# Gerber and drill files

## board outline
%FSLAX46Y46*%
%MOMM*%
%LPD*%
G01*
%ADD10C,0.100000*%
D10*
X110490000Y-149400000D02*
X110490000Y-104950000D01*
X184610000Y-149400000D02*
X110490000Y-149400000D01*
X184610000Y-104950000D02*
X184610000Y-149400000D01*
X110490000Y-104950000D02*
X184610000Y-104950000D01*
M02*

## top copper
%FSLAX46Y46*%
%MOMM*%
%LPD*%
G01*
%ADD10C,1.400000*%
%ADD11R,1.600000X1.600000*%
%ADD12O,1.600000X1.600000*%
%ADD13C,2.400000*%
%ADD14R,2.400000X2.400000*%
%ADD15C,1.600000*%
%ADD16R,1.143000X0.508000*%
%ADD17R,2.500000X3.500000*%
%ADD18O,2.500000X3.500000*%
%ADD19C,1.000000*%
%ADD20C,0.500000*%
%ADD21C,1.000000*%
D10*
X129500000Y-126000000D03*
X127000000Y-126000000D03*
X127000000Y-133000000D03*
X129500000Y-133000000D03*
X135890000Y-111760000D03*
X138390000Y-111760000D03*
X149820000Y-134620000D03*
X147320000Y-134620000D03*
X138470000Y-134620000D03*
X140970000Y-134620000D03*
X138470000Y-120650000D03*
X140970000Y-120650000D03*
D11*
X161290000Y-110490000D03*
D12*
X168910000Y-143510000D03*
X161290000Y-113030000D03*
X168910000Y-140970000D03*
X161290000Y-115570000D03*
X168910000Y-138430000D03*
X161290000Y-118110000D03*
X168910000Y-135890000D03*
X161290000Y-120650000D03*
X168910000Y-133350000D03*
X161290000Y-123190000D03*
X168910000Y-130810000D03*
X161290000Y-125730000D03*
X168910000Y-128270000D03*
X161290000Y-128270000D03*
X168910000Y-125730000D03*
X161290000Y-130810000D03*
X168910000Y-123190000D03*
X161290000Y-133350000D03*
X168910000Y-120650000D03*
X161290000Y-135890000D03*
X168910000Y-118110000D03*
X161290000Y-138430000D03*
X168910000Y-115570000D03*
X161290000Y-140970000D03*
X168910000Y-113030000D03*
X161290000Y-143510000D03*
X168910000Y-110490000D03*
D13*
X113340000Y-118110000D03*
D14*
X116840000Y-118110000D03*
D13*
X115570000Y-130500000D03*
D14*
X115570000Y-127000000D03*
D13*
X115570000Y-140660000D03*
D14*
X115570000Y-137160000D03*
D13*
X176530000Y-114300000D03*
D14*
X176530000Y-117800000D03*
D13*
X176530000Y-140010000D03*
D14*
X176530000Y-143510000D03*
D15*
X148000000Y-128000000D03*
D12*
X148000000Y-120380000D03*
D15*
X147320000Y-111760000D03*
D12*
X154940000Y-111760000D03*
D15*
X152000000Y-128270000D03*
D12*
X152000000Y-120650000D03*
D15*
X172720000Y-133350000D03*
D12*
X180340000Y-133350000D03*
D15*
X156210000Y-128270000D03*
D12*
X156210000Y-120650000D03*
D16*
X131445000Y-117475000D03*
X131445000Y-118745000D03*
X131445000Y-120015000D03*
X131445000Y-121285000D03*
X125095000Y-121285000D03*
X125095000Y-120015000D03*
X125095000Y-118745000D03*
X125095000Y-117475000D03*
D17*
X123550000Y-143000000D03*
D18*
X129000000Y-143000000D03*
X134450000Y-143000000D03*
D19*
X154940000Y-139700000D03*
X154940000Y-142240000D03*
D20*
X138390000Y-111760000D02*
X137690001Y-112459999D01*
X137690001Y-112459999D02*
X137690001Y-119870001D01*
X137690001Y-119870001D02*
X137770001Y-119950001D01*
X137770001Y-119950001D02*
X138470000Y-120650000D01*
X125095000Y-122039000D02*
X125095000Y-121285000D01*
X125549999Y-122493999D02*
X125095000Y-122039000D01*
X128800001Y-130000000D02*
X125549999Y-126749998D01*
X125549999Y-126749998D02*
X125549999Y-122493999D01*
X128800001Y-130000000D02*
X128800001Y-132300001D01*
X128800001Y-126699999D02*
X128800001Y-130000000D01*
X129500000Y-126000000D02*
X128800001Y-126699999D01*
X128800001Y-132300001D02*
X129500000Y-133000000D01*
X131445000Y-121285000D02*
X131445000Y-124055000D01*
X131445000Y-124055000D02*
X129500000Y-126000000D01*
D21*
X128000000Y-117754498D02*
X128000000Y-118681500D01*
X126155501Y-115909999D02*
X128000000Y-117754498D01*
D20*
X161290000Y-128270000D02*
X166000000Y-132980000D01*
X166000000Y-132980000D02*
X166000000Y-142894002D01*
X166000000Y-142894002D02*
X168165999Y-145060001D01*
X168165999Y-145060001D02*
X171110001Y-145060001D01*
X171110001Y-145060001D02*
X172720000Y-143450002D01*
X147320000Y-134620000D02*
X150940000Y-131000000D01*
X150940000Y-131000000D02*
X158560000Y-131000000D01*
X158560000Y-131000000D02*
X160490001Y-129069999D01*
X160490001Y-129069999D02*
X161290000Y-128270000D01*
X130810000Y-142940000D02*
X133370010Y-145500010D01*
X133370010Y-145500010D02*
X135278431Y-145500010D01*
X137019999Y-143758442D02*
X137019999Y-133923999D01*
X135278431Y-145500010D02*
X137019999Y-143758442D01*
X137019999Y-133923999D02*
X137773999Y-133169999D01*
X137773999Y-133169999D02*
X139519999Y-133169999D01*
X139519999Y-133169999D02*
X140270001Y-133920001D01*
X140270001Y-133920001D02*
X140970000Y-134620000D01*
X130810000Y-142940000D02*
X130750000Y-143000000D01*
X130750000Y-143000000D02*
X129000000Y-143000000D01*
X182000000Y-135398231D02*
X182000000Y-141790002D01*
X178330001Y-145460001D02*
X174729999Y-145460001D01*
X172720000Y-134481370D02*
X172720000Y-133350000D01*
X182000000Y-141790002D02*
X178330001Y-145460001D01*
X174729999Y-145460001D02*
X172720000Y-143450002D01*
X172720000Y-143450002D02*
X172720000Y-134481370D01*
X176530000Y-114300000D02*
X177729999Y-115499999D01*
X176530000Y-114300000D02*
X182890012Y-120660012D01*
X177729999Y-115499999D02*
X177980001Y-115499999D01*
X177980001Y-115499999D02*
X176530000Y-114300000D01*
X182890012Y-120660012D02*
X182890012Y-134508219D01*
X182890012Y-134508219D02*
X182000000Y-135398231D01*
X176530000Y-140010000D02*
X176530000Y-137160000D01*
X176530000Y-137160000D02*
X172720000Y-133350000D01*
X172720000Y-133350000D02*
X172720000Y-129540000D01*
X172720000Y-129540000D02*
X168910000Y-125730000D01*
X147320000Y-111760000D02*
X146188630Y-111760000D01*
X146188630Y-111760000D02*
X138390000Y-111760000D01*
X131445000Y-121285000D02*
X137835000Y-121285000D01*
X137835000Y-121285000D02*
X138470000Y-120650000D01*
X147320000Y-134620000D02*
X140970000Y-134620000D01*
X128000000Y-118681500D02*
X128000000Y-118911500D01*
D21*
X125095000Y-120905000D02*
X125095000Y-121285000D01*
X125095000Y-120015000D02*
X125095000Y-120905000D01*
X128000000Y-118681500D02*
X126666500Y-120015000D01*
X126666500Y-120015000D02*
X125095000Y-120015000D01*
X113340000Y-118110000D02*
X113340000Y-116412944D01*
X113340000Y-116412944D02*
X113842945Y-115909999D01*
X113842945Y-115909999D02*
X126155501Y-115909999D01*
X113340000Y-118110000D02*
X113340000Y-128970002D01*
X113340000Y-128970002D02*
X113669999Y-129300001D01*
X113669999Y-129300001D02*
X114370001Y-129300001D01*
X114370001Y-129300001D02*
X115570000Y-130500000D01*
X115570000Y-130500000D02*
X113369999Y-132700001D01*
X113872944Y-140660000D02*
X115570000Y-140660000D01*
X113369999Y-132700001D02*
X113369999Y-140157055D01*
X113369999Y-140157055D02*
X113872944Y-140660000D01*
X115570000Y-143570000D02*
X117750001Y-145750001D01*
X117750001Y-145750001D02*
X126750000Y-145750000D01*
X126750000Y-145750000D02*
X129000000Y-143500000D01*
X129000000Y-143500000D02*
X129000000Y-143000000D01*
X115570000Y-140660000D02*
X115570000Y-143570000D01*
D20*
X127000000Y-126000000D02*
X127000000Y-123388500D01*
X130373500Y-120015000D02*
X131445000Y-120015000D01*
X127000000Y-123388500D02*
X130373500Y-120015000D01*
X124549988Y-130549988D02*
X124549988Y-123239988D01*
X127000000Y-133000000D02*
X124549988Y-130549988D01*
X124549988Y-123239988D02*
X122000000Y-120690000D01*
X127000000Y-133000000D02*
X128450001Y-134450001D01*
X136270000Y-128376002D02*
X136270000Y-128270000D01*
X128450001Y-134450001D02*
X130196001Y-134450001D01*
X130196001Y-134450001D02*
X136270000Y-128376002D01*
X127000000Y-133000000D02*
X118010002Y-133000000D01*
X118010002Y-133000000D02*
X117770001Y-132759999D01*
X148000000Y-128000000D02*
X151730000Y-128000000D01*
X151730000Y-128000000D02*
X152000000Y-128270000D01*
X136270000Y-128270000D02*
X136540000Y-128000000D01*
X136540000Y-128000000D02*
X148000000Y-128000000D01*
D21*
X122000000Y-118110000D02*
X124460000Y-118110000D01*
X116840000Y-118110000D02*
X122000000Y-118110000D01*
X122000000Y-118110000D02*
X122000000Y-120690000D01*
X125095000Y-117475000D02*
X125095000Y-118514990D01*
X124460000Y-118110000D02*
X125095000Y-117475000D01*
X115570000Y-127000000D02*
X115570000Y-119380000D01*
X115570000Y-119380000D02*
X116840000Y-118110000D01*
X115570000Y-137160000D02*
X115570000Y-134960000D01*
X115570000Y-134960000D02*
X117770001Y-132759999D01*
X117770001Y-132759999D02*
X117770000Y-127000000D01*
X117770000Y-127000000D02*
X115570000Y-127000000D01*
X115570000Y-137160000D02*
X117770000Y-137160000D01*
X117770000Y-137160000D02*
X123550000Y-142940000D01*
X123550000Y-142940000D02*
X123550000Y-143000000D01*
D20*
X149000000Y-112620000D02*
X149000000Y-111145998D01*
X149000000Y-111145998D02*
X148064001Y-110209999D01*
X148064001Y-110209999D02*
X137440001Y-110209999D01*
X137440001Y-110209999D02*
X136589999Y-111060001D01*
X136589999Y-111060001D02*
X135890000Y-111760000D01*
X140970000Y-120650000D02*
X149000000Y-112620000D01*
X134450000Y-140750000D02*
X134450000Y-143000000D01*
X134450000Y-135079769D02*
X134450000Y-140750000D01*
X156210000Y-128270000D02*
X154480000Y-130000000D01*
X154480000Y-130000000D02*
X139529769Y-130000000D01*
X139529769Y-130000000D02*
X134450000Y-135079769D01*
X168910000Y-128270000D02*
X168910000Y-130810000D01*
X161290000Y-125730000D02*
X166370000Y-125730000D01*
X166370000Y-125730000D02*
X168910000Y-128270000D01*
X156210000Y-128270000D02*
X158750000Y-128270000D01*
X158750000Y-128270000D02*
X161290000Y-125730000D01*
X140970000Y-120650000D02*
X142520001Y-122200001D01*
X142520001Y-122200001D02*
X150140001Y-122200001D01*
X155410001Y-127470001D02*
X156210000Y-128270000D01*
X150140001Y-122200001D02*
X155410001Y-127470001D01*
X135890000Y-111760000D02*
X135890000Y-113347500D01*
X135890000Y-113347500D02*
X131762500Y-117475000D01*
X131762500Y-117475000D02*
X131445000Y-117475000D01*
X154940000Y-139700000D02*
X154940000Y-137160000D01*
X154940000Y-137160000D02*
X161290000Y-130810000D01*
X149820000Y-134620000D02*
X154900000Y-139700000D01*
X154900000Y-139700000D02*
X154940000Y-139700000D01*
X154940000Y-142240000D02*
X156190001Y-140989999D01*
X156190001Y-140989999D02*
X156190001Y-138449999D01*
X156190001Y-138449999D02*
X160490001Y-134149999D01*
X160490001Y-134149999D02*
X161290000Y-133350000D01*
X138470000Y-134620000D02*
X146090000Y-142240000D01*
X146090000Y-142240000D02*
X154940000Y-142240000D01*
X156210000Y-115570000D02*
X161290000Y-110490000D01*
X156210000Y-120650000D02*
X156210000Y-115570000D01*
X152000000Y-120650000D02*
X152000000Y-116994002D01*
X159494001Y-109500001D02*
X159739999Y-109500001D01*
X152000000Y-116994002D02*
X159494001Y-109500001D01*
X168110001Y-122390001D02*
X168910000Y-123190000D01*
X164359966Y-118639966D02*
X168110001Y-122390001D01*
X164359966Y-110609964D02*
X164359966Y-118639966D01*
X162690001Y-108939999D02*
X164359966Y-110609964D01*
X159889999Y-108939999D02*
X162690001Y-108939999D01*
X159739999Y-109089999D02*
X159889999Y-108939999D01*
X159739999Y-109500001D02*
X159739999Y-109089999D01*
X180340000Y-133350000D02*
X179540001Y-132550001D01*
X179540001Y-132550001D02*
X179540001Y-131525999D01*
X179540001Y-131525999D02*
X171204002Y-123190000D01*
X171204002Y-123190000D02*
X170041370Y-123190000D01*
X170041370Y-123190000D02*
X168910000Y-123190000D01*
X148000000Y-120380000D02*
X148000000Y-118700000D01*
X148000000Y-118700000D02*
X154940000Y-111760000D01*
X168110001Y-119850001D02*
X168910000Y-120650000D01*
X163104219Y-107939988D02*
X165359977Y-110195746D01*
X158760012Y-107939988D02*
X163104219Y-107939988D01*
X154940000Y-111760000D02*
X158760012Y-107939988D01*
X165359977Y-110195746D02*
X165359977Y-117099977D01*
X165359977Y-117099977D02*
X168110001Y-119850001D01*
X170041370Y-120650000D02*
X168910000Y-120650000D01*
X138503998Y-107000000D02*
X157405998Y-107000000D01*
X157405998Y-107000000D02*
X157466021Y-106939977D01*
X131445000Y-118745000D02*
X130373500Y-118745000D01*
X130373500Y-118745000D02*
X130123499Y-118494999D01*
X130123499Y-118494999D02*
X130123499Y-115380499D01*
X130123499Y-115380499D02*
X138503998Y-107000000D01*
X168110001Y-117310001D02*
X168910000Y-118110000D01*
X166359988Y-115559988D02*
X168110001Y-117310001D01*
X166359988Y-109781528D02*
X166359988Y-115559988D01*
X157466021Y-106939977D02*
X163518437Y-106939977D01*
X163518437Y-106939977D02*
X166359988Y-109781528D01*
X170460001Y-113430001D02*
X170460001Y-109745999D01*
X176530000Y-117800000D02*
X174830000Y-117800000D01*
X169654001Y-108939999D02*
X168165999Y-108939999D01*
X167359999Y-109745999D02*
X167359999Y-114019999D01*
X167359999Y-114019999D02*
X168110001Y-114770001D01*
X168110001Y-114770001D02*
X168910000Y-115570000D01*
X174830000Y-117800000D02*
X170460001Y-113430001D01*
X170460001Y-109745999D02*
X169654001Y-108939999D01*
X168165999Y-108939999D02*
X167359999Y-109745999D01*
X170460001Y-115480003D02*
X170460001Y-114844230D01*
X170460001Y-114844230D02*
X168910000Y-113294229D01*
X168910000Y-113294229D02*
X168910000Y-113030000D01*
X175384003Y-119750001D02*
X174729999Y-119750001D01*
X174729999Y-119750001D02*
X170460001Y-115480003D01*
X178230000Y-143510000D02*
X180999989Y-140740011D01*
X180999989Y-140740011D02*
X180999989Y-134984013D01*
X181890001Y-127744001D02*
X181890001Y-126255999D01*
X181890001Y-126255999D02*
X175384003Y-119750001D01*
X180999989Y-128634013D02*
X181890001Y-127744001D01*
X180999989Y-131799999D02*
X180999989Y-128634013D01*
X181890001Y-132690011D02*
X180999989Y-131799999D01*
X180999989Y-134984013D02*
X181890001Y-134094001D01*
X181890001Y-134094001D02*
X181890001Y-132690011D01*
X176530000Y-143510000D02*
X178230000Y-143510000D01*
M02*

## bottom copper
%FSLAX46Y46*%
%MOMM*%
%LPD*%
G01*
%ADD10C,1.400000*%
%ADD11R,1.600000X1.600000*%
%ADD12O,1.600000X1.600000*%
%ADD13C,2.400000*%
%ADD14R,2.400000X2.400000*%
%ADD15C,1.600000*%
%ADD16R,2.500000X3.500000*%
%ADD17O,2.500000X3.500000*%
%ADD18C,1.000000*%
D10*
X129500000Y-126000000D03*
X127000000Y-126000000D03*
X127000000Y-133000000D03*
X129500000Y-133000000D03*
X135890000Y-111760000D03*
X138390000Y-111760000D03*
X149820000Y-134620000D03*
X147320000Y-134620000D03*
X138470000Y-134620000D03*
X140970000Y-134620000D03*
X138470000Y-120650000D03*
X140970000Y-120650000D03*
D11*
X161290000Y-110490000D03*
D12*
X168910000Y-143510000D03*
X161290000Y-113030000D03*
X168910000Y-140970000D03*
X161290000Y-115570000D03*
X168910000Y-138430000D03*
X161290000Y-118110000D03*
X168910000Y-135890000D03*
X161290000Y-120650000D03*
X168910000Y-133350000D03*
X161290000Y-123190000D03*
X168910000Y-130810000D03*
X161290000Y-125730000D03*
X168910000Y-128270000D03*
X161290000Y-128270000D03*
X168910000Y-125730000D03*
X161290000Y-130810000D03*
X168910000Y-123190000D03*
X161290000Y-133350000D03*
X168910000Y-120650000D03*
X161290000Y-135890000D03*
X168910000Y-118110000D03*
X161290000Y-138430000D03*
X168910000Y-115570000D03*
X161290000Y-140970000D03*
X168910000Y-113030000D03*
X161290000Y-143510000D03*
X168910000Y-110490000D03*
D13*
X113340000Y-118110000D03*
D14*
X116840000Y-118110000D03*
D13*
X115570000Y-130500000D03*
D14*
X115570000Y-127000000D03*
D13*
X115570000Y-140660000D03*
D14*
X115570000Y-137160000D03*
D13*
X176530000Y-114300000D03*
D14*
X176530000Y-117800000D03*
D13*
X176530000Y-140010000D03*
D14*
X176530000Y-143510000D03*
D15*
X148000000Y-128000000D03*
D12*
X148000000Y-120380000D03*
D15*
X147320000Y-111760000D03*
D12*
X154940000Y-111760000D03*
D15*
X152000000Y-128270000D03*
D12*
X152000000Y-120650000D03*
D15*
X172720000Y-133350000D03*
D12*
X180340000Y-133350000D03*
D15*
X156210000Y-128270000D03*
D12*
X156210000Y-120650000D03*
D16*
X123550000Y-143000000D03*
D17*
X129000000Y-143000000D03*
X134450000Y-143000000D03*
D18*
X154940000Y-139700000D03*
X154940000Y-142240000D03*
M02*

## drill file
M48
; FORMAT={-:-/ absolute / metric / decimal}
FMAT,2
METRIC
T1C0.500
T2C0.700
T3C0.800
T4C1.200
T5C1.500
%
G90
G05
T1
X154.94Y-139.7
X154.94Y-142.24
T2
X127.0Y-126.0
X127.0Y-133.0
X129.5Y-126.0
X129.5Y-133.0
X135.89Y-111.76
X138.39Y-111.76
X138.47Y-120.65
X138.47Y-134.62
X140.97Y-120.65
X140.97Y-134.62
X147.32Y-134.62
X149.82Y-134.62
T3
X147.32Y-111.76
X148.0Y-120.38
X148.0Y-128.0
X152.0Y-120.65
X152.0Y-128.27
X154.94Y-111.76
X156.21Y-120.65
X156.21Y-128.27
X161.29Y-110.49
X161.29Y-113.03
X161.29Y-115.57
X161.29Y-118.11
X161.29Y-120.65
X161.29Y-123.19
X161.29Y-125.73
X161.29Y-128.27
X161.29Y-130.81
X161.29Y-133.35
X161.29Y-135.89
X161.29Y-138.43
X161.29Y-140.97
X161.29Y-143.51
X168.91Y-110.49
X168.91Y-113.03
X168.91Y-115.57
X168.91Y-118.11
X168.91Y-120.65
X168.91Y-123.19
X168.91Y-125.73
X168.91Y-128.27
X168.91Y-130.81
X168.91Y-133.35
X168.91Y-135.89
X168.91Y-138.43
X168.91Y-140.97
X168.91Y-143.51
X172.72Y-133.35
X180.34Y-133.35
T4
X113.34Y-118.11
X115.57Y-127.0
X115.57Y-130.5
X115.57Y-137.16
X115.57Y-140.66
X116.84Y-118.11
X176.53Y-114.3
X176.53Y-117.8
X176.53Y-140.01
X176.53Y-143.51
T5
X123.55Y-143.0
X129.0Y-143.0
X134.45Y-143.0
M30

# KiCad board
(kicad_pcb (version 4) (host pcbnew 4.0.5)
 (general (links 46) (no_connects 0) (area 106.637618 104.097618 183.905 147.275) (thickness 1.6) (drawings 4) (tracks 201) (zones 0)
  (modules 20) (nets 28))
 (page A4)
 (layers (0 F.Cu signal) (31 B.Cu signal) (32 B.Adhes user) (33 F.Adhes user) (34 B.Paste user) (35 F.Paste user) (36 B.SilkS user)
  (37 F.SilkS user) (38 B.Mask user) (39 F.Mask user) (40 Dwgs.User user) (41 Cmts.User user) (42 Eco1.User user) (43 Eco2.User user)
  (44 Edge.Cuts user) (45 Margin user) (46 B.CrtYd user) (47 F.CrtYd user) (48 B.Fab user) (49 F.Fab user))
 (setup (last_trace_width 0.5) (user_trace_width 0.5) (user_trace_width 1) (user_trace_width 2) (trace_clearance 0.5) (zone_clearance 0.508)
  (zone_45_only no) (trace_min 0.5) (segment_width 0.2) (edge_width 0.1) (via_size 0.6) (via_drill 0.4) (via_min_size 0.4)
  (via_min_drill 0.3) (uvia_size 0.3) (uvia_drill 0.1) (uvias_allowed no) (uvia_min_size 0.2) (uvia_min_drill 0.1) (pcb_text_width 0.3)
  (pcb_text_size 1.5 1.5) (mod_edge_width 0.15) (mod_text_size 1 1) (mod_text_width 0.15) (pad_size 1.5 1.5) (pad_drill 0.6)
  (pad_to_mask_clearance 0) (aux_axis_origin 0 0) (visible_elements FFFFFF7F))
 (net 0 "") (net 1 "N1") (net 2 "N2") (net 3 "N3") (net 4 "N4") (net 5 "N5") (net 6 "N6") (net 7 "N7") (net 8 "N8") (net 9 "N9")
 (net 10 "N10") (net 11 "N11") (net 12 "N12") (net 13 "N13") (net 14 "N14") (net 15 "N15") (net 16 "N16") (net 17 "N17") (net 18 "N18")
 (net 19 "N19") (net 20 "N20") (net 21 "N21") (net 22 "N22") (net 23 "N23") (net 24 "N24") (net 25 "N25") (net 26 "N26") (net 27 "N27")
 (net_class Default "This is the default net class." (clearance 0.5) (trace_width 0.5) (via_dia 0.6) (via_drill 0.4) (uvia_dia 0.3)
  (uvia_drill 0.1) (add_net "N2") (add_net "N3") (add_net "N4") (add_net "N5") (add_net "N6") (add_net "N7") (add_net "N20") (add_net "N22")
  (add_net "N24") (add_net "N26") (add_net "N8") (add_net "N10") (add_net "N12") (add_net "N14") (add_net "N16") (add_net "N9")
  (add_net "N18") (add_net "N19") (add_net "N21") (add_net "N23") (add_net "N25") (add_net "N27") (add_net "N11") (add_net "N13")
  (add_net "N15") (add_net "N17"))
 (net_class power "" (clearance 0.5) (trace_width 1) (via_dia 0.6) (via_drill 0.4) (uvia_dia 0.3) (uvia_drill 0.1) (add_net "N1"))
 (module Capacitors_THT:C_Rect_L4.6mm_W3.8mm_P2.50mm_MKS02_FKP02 (layer F.Cu) (at 129.5 126 180)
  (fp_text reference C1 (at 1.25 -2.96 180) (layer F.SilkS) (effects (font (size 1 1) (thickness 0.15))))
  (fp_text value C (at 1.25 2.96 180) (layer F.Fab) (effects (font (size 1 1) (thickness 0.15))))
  (pad 1 thru_hole circle (at 0 0 180) (size 1.4 1.4) (drill 0.7) (layers *.Cu *.Mask) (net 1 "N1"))
  (pad 2 thru_hole circle (at 2.5 0 180) (size 1.4 1.4) (drill 0.7) (layers *.Cu *.Mask) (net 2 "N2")))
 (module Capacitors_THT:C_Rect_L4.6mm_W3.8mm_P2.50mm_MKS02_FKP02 (layer F.Cu) (at 127 133)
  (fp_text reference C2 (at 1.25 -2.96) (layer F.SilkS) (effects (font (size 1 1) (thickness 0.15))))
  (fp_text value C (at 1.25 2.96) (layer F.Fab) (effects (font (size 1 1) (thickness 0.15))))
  (pad 1 thru_hole circle (at 0 0) (size 1.4 1.4) (drill 0.7) (layers *.Cu *.Mask) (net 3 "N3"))
  (pad 2 thru_hole circle (at 2.5 0) (size 1.4 1.4) (drill 0.7) (layers *.Cu *.Mask) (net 1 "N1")))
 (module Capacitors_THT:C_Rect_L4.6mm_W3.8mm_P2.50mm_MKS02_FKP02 (layer F.Cu) (at 135.89 111.76)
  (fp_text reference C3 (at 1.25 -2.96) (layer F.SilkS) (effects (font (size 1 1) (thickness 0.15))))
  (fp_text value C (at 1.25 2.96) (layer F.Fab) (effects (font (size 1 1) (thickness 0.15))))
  (pad 1 thru_hole circle (at 0 0) (size 1.4 1.4) (drill 0.7) (layers *.Cu *.Mask) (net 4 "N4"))
  (pad 2 thru_hole circle (at 2.5 0) (size 1.4 1.4) (drill 0.7) (layers *.Cu *.Mask) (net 1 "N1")))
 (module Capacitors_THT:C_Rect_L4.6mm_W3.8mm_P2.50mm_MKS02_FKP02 (layer F.Cu) (at 149.82 134.62 180)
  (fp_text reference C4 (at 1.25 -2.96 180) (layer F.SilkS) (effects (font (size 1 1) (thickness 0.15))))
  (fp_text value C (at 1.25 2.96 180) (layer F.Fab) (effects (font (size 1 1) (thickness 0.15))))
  (pad 1 thru_hole circle (at 0 0 180) (size 1.4 1.4) (drill 0.7) (layers *.Cu *.Mask) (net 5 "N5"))
  (pad 2 thru_hole circle (at 2.5 0 180) (size 1.4 1.4) (drill 0.7) (layers *.Cu *.Mask) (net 1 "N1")))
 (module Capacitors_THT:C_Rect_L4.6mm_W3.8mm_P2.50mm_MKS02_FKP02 (layer F.Cu) (at 138.47 134.62)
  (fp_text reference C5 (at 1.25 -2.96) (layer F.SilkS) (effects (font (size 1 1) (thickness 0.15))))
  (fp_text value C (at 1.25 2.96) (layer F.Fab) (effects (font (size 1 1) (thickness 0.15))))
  (pad 1 thru_hole circle (at 0 0) (size 1.4 1.4) (drill 0.7) (layers *.Cu *.Mask) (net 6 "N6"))
  (pad 2 thru_hole circle (at 2.5 0) (size 1.4 1.4) (drill 0.7) (layers *.Cu *.Mask) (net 1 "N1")))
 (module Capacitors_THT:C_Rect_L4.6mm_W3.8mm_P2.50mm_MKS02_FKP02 (layer F.Cu) (at 138.47 120.65)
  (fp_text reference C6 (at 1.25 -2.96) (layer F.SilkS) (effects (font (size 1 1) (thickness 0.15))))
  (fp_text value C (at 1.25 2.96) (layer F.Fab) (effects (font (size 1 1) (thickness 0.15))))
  (pad 1 thru_hole circle (at 0 0) (size 1.4 1.4) (drill 0.7) (layers *.Cu *.Mask) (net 1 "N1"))
  (pad 2 thru_hole circle (at 2.5 0) (size 1.4 1.4) (drill 0.7) (layers *.Cu *.Mask) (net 4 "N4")))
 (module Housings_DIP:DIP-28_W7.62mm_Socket (layer F.Cu) (at 161.29 110.49)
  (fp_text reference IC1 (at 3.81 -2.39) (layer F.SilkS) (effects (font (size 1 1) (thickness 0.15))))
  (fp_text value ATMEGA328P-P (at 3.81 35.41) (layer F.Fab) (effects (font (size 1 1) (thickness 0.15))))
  (pad 1 thru_hole rect (at 0 0) (size 1.6 1.6) (drill 0.8) (layers *.Cu *.Mask) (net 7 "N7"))
  (pad 15 thru_hole oval (at 7.62 33.02) (size 1.6 1.6) (drill 0.8) (layers *.Cu *.Mask) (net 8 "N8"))
  (pad 2 thru_hole oval (at 0 2.54) (size 1.6 1.6) (drill 0.8) (layers *.Cu *.Mask) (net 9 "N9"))
  (pad 16 thru_hole oval (at 7.62 30.48) (size 1.6 1.6) (drill 0.8) (layers *.Cu *.Mask) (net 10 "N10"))
  (pad 3 thru_hole oval (at 0 5.08) (size 1.6 1.6) (drill 0.8) (layers *.Cu *.Mask) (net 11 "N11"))
  (pad 17 thru_hole oval (at 7.62 27.94) (size 1.6 1.6) (drill 0.8) (layers *.Cu *.Mask) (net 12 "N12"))
  (pad 4 thru_hole oval (at 0 7.62) (size 1.6 1.6) (drill 0.8) (layers *.Cu *.Mask) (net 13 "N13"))
  (pad 18 thru_hole oval (at 7.62 25.4) (size 1.6 1.6) (drill 0.8) (layers *.Cu *.Mask) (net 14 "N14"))
  (pad 5 thru_hole oval (at 0 10.16) (size 1.6 1.6) (drill 0.8) (layers *.Cu *.Mask) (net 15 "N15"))
  (pad 19 thru_hole oval (at 7.62 22.86) (size 1.6 1.6) (drill 0.8) (layers *.Cu *.Mask) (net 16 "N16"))
  (pad 6 thru_hole oval (at 0 12.7) (size 1.6 1.6) (drill 0.8) (layers *.Cu *.Mask) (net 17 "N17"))
  (pad 20 thru_hole oval (at 7.62 20.32) (size 1.6 1.6) (drill 0.8) (layers *.Cu *.Mask) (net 4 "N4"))
  (pad 7 thru_hole oval (at 0 15.24) (size 1.6 1.6) (drill 0.8) (layers *.Cu *.Mask) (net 4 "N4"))
  (pad 21 thru_hole oval (at 7.62 17.78) (size 1.6 1.6) (drill 0.8) (layers *.Cu *.Mask) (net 4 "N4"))
  (pad 8 thru_hole oval (at 0 17.78) (size 1.6 1.6) (drill 0.8) (layers *.Cu *.Mask) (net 1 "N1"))
  (pad 22 thru_hole oval (at 7.62 15.24) (size 1.6 1.6) (drill 0.8) (layers *.Cu *.Mask) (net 1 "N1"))
  (pad 9 thru_hole oval (at 0 20.32) (size 1.6 1.6) (drill 0.8) (layers *.Cu *.Mask) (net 5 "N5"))
  (pad 23 thru_hole oval (at 7.62 12.7) (size 1.6 1.6) (drill 0.8) (layers *.Cu *.Mask) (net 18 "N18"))
  (pad 10 thru_hole oval (at 0 22.86) (size 1.6 1.6) (drill 0.8) (layers *.Cu *.Mask) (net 6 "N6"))
  (pad 24 thru_hole oval (at 7.62 10.16) (size 1.6 1.6) (drill 0.8) (layers *.Cu *.Mask) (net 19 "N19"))
  (pad 11 thru_hole oval (at 0 25.4) (size 1.6 1.6) (drill 0.8) (layers *.Cu *.Mask) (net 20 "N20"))
  (pad 25 thru_hole oval (at 7.62 7.62) (size 1.6 1.6) (drill 0.8) (layers *.Cu *.Mask) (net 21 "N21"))
  (pad 12 thru_hole oval (at 0 27.94) (size 1.6 1.6) (drill 0.8) (layers *.Cu *.Mask) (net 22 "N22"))
  (pad 26 thru_hole oval (at 7.62 5.08) (size 1.6 1.6) (drill 0.8) (layers *.Cu *.Mask) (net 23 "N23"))
  (pad 13 thru_hole oval (at 0 30.48) (size 1.6 1.6) (drill 0.8) (layers *.Cu *.Mask) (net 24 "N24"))
  (pad 27 thru_hole oval (at 7.62 2.54) (size 1.6 1.6) (drill 0.8) (layers *.Cu *.Mask) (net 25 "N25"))
  (pad 14 thru_hole oval (at 0 33.02) (size 1.6 1.6) (drill 0.8) (layers *.Cu *.Mask) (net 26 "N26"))
  (pad 28 thru_hole oval (at 7.62 0) (size 1.6 1.6) (drill 0.8) (layers *.Cu *.Mask) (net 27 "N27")))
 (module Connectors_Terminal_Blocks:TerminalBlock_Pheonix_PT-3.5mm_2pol (layer F.Cu) (at 116.84 118.11 180)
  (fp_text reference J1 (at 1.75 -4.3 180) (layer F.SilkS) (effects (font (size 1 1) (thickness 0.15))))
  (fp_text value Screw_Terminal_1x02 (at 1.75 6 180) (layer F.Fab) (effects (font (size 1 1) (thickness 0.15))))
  (pad 2 thru_hole circle (at 3.5 0 180) (size 2.4 2.4) (drill 1.2) (layers *.Cu *.Mask) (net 1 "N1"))
  (pad 1 thru_hole rect (at 0 0 180) (size 2.4 2.4) (drill 1.2) (layers *.Cu *.Mask) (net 3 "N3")))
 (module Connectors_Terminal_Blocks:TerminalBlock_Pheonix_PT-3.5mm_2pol (layer F.Cu) (at 115.57 127 270)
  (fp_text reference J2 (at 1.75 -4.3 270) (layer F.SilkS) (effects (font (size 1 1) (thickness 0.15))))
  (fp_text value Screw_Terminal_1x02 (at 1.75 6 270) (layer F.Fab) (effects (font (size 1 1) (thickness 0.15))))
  (pad 2 thru_hole circle (at 3.5 0 270) (size 2.4 2.4) (drill 1.2) (layers *.Cu *.Mask) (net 1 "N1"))
  (pad 1 thru_hole rect (at 0 0 270) (size 2.4 2.4) (drill 1.2) (layers *.Cu *.Mask) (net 3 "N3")))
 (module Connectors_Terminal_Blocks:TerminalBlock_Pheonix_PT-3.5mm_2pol (layer F.Cu) (at 115.57 137.16 270)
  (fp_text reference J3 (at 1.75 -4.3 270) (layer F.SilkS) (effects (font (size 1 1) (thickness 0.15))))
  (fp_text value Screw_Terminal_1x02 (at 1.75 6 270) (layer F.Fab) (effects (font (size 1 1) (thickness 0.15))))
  (pad 2 thru_hole circle (at 3.5 0 270) (size 2.4 2.4) (drill 1.2) (layers *.Cu *.Mask) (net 1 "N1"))
  (pad 1 thru_hole rect (at 0 0 270) (size 2.4 2.4) (drill 1.2) (layers *.Cu *.Mask) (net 3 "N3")))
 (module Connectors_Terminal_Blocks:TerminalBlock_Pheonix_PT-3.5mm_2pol (layer F.Cu) (at 176.53 117.8 90)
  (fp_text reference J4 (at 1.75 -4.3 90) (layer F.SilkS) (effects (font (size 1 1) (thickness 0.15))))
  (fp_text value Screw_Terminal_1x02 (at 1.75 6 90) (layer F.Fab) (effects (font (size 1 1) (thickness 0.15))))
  (pad 2 thru_hole circle (at 3.5 0 90) (size 2.4 2.4) (drill 1.2) (layers *.Cu *.Mask) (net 1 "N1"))
  (pad 1 thru_hole rect (at 0 0 90) (size 2.4 2.4) (drill 1.2) (layers *.Cu *.Mask) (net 23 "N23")))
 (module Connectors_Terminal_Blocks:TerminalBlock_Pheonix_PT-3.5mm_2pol (layer F.Cu) (at 176.53 143.51 90)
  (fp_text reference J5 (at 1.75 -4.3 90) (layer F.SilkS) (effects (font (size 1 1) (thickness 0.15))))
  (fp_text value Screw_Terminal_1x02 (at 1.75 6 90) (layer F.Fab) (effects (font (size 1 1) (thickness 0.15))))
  (pad 2 thru_hole circle (at 3.5 0 90) (size 2.4 2.4) (drill 1.2) (layers *.Cu *.Mask) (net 1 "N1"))
  (pad 1 thru_hole rect (at 0 0 90) (size 2.4 2.4) (drill 1.2) (layers *.Cu *.Mask) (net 25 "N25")))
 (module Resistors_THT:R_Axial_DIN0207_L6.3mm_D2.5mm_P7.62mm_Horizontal (layer F.Cu) (at 148 128 90)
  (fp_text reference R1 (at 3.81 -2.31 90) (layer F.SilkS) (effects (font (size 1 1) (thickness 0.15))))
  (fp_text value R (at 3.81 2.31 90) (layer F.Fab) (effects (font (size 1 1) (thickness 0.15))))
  (pad 1 thru_hole circle (at 0 0 90) (size 1.6 1.6) (drill 0.8) (layers *.Cu *.Mask) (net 3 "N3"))
  (pad 2 thru_hole oval (at 7.62 0 90) (size 1.6 1.6) (drill 0.8) (layers *.Cu *.Mask) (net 19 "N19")))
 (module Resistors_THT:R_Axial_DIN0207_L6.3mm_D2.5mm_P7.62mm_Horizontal (layer F.Cu) (at 147.32 111.76)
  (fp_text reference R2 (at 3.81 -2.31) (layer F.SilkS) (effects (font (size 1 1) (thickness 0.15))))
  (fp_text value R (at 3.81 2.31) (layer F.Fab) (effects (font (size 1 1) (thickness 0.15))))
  (pad 1 thru_hole circle (at 0 0) (size 1.6 1.6) (drill 0.8) (layers *.Cu *.Mask) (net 1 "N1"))
  (pad 2 thru_hole oval (at 7.62 0) (size 1.6 1.6) (drill 0.8) (layers *.Cu *.Mask) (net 19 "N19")))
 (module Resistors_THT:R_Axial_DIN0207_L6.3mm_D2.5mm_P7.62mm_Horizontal (layer F.Cu) (at 152 128.27 90)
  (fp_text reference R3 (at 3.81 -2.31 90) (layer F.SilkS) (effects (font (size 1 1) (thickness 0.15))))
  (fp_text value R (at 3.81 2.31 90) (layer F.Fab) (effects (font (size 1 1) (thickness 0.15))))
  (pad 1 thru_hole circle (at 0 0 90) (size 1.6 1.6) (drill 0.8) (layers *.Cu *.Mask) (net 3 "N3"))
  (pad 2 thru_hole oval (at 7.62 0 90) (size 1.6 1.6) (drill 0.8) (layers *.Cu *.Mask) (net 18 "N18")))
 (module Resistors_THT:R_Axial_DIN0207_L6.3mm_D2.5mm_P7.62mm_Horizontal (layer F.Cu) (at 172.72 133.35)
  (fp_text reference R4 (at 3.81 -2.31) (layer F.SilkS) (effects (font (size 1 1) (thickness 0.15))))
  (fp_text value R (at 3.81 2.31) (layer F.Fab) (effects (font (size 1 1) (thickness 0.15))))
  (pad 1 thru_hole circle (at 0 0) (size 1.6 1.6) (drill 0.8) (layers *.Cu *.Mask) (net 1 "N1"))
  (pad 2 thru_hole oval (at 7.62 0) (size 1.6 1.6) (drill 0.8) (layers *.Cu *.Mask) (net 18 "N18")))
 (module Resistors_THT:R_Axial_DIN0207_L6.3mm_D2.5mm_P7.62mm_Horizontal (layer F.Cu) (at 156.21 128.27 90)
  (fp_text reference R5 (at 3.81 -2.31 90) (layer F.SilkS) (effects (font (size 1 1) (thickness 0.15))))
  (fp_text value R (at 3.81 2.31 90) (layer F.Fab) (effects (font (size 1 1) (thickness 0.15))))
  (pad 1 thru_hole circle (at 0 0 90) (size 1.6 1.6) (drill 0.8) (layers *.Cu *.Mask) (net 4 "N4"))
  (pad 2 thru_hole oval (at 7.62 0 90) (size 1.6 1.6) (drill 0.8) (layers *.Cu *.Mask) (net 7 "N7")))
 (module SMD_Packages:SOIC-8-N (layer F.Cu) (at 128.27 119.38 270)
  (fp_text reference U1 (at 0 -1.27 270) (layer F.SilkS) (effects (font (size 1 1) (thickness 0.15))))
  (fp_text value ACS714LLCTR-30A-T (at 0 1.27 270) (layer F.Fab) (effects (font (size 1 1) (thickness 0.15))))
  (pad 8 smd rect (at -1.905 -3.175 270) (size 0.508 1.143) (layers F.Cu F.Paste F.Mask) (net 4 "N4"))
  (pad 7 smd rect (at -0.635 -3.175 270) (size 0.508 1.143) (layers F.Cu F.Paste F.Mask) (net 21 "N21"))
  (pad 6 smd rect (at 0.635 -3.175 270) (size 0.508 1.143) (layers F.Cu F.Paste F.Mask) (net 2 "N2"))
  (pad 5 smd rect (at 1.905 -3.175 270) (size 0.508 1.143) (layers F.Cu F.Paste F.Mask) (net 1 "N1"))
  (pad 4 smd rect (at 1.905 3.175 270) (size 0.508 1.143) (layers F.Cu F.Paste F.Mask) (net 1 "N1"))
  (pad 3 smd rect (at 0.635 3.175 270) (size 0.508 1.143) (layers F.Cu F.Paste F.Mask) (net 1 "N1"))
  (pad 2 smd rect (at -0.635 3.175 270) (size 0.508 1.143) (layers F.Cu F.Paste F.Mask) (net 3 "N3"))
  (pad 1 smd rect (at -1.905 3.175 270) (size 0.508 1.143) (layers F.Cu F.Paste F.Mask) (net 3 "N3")))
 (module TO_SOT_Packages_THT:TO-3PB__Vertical (layer F.Cu) (at 123.55 143)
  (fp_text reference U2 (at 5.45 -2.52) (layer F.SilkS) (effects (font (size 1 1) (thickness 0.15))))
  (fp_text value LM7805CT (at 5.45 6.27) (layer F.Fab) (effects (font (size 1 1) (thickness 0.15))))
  (pad 1 thru_hole rect (at 0 0) (size 2.5 3.5) (drill 1.5) (layers *.Cu *.Mask) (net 3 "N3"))
  (pad 2 thru_hole oval (at 5.45 0) (size 2.5 3.5) (drill 1.5) (layers *.Cu *.Mask) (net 1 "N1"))
  (pad 3 thru_hole oval (at 10.9 0) (size 2.5 3.5) (drill 1.5) (layers *.Cu *.Mask) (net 4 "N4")))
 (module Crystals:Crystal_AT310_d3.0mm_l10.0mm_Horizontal (layer F.Cu) (at 154.94 139.7 270)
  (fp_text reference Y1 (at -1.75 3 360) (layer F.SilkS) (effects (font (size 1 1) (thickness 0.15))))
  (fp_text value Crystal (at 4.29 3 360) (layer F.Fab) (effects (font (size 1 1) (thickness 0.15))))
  (pad 1 thru_hole circle (at 0 0 270) (size 1 1) (drill 0.5) (layers *.Cu *.Mask) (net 5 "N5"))
  (pad 2 thru_hole circle (at 2.54 0 270) (size 1 1) (drill 0.5) (layers *.Cu *.Mask) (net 6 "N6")))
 (gr_line (start 110.49 149.4) (end 110.49 104.95) (angle 90) (layer Edge.Cuts) (width 0.1))
 (gr_line (start 184.61 149.4) (end 110.49 149.4) (angle 90) (layer Edge.Cuts) (width 0.1))
 (gr_line (start 184.61 104.95) (end 184.61 149.4) (angle 90) (layer Edge.Cuts) (width 0.1))
 (gr_line (start 110.49 104.95) (end 184.61 104.95) (angle 90) (layer Edge.Cuts) (width 0.1))
 (segment (start 138.39 111.76) (end 137.690001 112.459999) (width 0.5) (layer F.Cu) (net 1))
 (segment (start 137.690001 112.459999) (end 137.690001 119.870001) (width 0.5) (layer F.Cu) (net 1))
 (segment (start 137.690001 119.870001) (end 137.770001 119.950001) (width 0.5) (layer F.Cu) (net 1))
 (segment (start 137.770001 119.950001) (end 138.47 120.65) (width 0.5) (layer F.Cu) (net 1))
 (segment (start 125.095 122.039) (end 125.095 121.285) (width 0.5) (layer F.Cu) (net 1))
 (segment (start 125.549999 122.493999) (end 125.095 122.039) (width 0.5) (layer F.Cu) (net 1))
 (segment (start 128.800001 130) (end 125.549999 126.749998) (width 0.5) (layer F.Cu) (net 1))
 (segment (start 125.549999 126.749998) (end 125.549999 122.493999) (width 0.5) (layer F.Cu) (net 1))
 (segment (start 128.800001 130) (end 128.800001 132.300001) (width 0.5) (layer F.Cu) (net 1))
 (segment (start 128.800001 126.699999) (end 128.800001 130) (width 0.5) (layer F.Cu) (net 1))
 (segment (start 129.5 126) (end 128.800001 126.699999) (width 0.5) (layer F.Cu) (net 1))
 (segment (start 128.800001 132.300001) (end 129.5 133) (width 0.5) (layer F.Cu) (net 1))
 (segment (start 131.445 121.285) (end 131.445 124.055) (width 0.5) (layer F.Cu) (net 1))
 (segment (start 131.445 124.055) (end 129.5 126) (width 0.5) (layer F.Cu) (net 1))
 (segment (start 128 117.754498) (end 128 118.6815) (width 1) (layer F.Cu) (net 1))
 (segment (start 126.155501 115.909999) (end 128 117.754498) (width 1) (layer F.Cu) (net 1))
 (segment (start 161.29 128.27) (end 166 132.98) (width 0.5) (layer F.Cu) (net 1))
 (segment (start 166 132.98) (end 166 142.894002) (width 0.5) (layer F.Cu) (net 1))
 (segment (start 166 142.894002) (end 168.165999 145.060001) (width 0.5) (layer F.Cu) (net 1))
 (segment (start 168.165999 145.060001) (end 171.110001 145.060001) (width 0.5) (layer F.Cu) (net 1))
 (segment (start 171.110001 145.060001) (end 172.72 143.450002) (width 0.5) (layer F.Cu) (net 1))
 (segment (start 147.32 134.62) (end 150.94 131) (width 0.5) (layer F.Cu) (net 1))
 (segment (start 150.94 131) (end 158.56 131) (width 0.5) (layer F.Cu) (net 1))
 (segment (start 158.56 131) (end 160.490001 129.069999) (width 0.5) (layer F.Cu) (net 1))
 (segment (start 160.490001 129.069999) (end 161.29 128.27) (width 0.5) (layer F.Cu) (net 1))
 (segment (start 130.81 142.94) (end 133.37001 145.50001) (width 0.5) (layer F.Cu) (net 1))
 (segment (start 133.37001 145.50001) (end 135.278431 145.50001) (width 0.5) (layer F.Cu) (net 1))
 (segment (start 137.019999 143.758442) (end 137.019999 133.923999) (width 0.5) (layer F.Cu) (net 1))
 (segment (start 135.278431 145.50001) (end 137.019999 143.758442) (width 0.5) (layer F.Cu) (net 1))
 (segment (start 137.019999 133.923999) (end 137.773999 133.169999) (width 0.5) (layer F.Cu) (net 1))
 (segment (start 137.773999 133.169999) (end 139.519999 133.169999) (width 0.5) (layer F.Cu) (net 1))
 (segment (start 139.519999 133.169999) (end 140.270001 133.920001) (width 0.5) (layer F.Cu) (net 1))
 (segment (start 140.270001 133.920001) (end 140.97 134.62) (width 0.5) (layer F.Cu) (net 1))
 (segment (start 130.81 142.94) (end 130.75 143) (width 0.5) (layer F.Cu) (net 1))
 (segment (start 130.75 143) (end 129 143) (width 0.5) (layer F.Cu) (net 1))
 (segment (start 182 135.398231) (end 182 141.790002) (width 0.5) (layer F.Cu) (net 1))
 (segment (start 178.330001 145.460001) (end 174.729999 145.460001) (width 0.5) (layer F.Cu) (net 1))
 (segment (start 172.72 134.48137) (end 172.72 133.35) (width 0.5) (layer F.Cu) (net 1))
 (segment (start 182 141.790002) (end 178.330001 145.460001) (width 0.5) (layer F.Cu) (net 1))
 (segment (start 174.729999 145.460001) (end 172.72 143.450002) (width 0.5) (layer F.Cu) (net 1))
 (segment (start 172.72 143.450002) (end 172.72 134.48137) (width 0.5) (layer F.Cu) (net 1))
 (segment (start 176.53 114.3) (end 177.729999 115.499999) (width 0.5) (layer F.Cu) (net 1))
 (segment (start 176.53 114.3) (end 182.890012 120.660012) (width 0.5) (layer F.Cu) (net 1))
 (segment (start 177.729999 115.499999) (end 177.980001 115.499999) (width 0.5) (layer F.Cu) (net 1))
 (segment (start 177.980001 115.499999) (end 176.53 114.3) (width 0.5) (layer F.Cu) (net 1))
 (segment (start 182.890012 120.660012) (end 182.890012 134.508219) (width 0.5) (layer F.Cu) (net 1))
 (segment (start 182.890012 134.508219) (end 182 135.398231) (width 0.5) (layer F.Cu) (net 1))
 (segment (start 176.53 140.01) (end 176.53 137.16) (width 0.5) (layer F.Cu) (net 1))
 (segment (start 176.53 137.16) (end 172.72 133.35) (width 0.5) (layer F.Cu) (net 1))
 (segment (start 172.72 133.35) (end 172.72 129.54) (width 0.5) (layer F.Cu) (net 1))
 (segment (start 172.72 129.54) (end 168.91 125.73) (width 0.5) (layer F.Cu) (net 1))
 (segment (start 147.32 111.76) (end 146.18863 111.76) (width 0.5) (layer F.Cu) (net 1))
 (segment (start 146.18863 111.76) (end 138.39 111.76) (width 0.5) (layer F.Cu) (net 1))
 (segment (start 131.445 121.285) (end 137.835 121.285) (width 0.5) (layer F.Cu) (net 1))
 (segment (start 137.835 121.285) (end 138.47 120.65) (width 0.5) (layer F.Cu) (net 1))
 (segment (start 147.32 134.62) (end 140.97 134.62) (width 0.5) (layer F.Cu) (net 1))
 (segment (start 128 118.6815) (end 128 118.9115) (width 0.5) (layer F.Cu) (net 1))
 (segment (start 125.095 120.905) (end 125.095 121.285) (width 1) (layer F.Cu) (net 1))
 (segment (start 125.095 120.015) (end 125.095 120.905) (width 1) (layer F.Cu) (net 1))
 (segment (start 128 118.6815) (end 126.6665 120.015) (width 1) (layer F.Cu) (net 1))
 (segment (start 126.6665 120.015) (end 125.095 120.015) (width 1) (layer F.Cu) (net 1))
 (segment (start 113.34 118.11) (end 113.34 116.412944) (width 1) (layer F.Cu) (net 1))
 (segment (start 113.34 116.412944) (end 113.842945 115.909999) (width 1) (layer F.Cu) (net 1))
 (segment (start 113.842945 115.909999) (end 126.155501 115.909999) (width 1) (layer F.Cu) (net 1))
 (segment (start 113.34 118.11) (end 113.34 128.970002) (width 1) (layer F.Cu) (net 1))
 (segment (start 113.34 128.970002) (end 113.669999 129.300001) (width 1) (layer F.Cu) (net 1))
 (segment (start 113.669999 129.300001) (end 114.370001 129.300001) (width 1) (layer F.Cu) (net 1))
 (segment (start 114.370001 129.300001) (end 115.57 130.5) (width 1) (layer F.Cu) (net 1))
 (segment (start 115.57 130.5) (end 113.369999 132.700001) (width 1) (layer F.Cu) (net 1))
 (segment (start 113.872944 140.66) (end 115.57 140.66) (width 1) (layer F.Cu) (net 1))
 (segment (start 113.369999 132.700001) (end 113.369999 140.157055) (width 1) (layer F.Cu) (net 1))
 (segment (start 113.369999 140.157055) (end 113.872944 140.66) (width 1) (layer F.Cu) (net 1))
 (segment (start 115.57 143.57) (end 117.750001 145.750001) (width 1) (layer F.Cu) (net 1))
 (segment (start 117.750001 145.750001) (end 126.75 145.75) (width 1) (layer F.Cu) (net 1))
 (segment (start 126.75 145.75) (end 129 143.5) (width 1) (layer F.Cu) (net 1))
 (segment (start 129 143.5) (end 129 143) (width 1) (layer F.Cu) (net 1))
 (segment (start 115.57 140.66) (end 115.57 143.57) (width 1) (layer F.Cu) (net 1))
 (segment (start 127 126) (end 127 123.3885) (width 0.5) (layer F.Cu) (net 2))
 (segment (start 130.3735 120.015) (end 131.445 120.015) (width 0.5) (layer F.Cu) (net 2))
 (segment (start 127 123.3885) (end 130.3735 120.015) (width 0.5) (layer F.Cu) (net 2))
 (segment (start 124.549988 130.549988) (end 124.549988 123.239988) (width 0.5) (layer F.Cu) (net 3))
 (segment (start 127 133) (end 124.549988 130.549988) (width 0.5) (layer F.Cu) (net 3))
 (segment (start 124.549988 123.239988) (end 122 120.69) (width 0.5) (layer F.Cu) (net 3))
 (segment (start 127 133) (end 128.450001 134.450001) (width 0.5) (layer F.Cu) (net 3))
 (segment (start 136.27 128.376002) (end 136.27 128.27) (width 0.5) (layer F.Cu) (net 3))
 (segment (start 128.450001 134.450001) (end 130.196001 134.450001) (width 0.5) (layer F.Cu) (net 3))
 (segment (start 130.196001 134.450001) (end 136.27 128.376002) (width 0.5) (layer F.Cu) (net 3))
 (segment (start 127 133) (end 118.010002 133) (width 0.5) (layer F.Cu) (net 3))
 (segment (start 118.010002 133) (end 117.770001 132.759999) (width 0.5) (layer F.Cu) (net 3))
 (segment (start 148 128) (end 151.73 128) (width 0.5) (layer F.Cu) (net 3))
 (segment (start 151.73 128) (end 152 128.27) (width 0.5) (layer F.Cu) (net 3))
 (segment (start 136.27 128.27) (end 136.54 128) (width 0.5) (layer F.Cu) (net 3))
 (segment (start 136.54 128) (end 148 128) (width 0.5) (layer F.Cu) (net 3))
 (segment (start 122 118.11) (end 124.46 118.11) (width 1) (layer F.Cu) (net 3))
 (segment (start 116.84 118.11) (end 122 118.11) (width 1) (layer F.Cu) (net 3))
 (segment (start 122 118.11) (end 122 120.69) (width 1) (layer F.Cu) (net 3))
 (segment (start 125.095 117.475) (end 125.095 118.51499) (width 1) (layer F.Cu) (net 3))
 (segment (start 124.46 118.11) (end 125.095 117.475) (width 1) (layer F.Cu) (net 3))
 (segment (start 115.57 127) (end 115.57 119.38) (width 1) (layer F.Cu) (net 3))
 (segment (start 115.57 119.38) (end 116.84 118.11) (width 1) (layer F.Cu) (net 3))
 (segment (start 115.57 137.16) (end 115.57 134.96) (width 1) (layer F.Cu) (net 3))
 (segment (start 115.57 134.96) (end 117.770001 132.759999) (width 1) (layer F.Cu) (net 3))
 (segment (start 117.770001 132.759999) (end 117.77 127) (width 1) (layer F.Cu) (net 3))
 (segment (start 117.77 127) (end 115.57 127) (width 1) (layer F.Cu) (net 3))
 (segment (start 115.57 137.16) (end 117.77 137.16) (width 1) (layer F.Cu) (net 3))
 (segment (start 117.77 137.16) (end 123.55 142.94) (width 1) (layer F.Cu) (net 3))
 (segment (start 123.55 142.94) (end 123.55 143) (width 1) (layer F.Cu) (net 3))
 (segment (start 149 112.62) (end 149 111.145998) (width 0.5) (layer F.Cu) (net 4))
 (segment (start 149 111.145998) (end 148.064001 110.209999) (width 0.5) (layer F.Cu) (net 4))
 (segment (start 148.064001 110.209999) (end 137.440001 110.209999) (width 0.5) (layer F.Cu) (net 4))
 (segment (start 137.440001 110.209999) (end 136.589999 111.060001) (width 0.5) (layer F.Cu) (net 4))
 (segment (start 136.589999 111.060001) (end 135.89 111.76) (width 0.5) (layer F.Cu) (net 4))
 (segment (start 140.97 120.65) (end 149 112.62) (width 0.5) (layer F.Cu) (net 4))
 (segment (start 134.45 140.75) (end 134.45 143) (width 0.5) (layer F.Cu) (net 4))
 (segment (start 134.45 135.079769) (end 134.45 140.75) (width 0.5) (layer F.Cu) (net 4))
 (segment (start 156.21 128.27) (end 154.48 130) (width 0.5) (layer F.Cu) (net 4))
 (segment (start 154.48 130) (end 139.529769 130) (width 0.5) (layer F.Cu) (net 4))
 (segment (start 139.529769 130) (end 134.45 135.079769) (width 0.5) (layer F.Cu) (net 4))
 (segment (start 168.91 128.27) (end 168.91 130.81) (width 0.5) (layer F.Cu) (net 4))
 (segment (start 161.29 125.73) (end 166.37 125.73) (width 0.5) (layer F.Cu) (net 4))
 (segment (start 166.37 125.73) (end 168.91 128.27) (width 0.5) (layer F.Cu) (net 4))
 (segment (start 156.21 128.27) (end 158.75 128.27) (width 0.5) (layer F.Cu) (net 4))
 (segment (start 158.75 128.27) (end 161.29 125.73) (width 0.5) (layer F.Cu) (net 4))
 (segment (start 140.97 120.65) (end 142.520001 122.200001) (width 0.5) (layer F.Cu) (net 4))
 (segment (start 142.520001 122.200001) (end 150.140001 122.200001) (width 0.5) (layer F.Cu) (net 4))
 (segment (start 155.410001 127.470001) (end 156.21 128.27) (width 0.5) (layer F.Cu) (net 4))
 (segment (start 150.140001 122.200001) (end 155.410001 127.470001) (width 0.5) (layer F.Cu) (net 4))
 (segment (start 135.89 111.76) (end 135.89 113.3475) (width 0.5) (layer F.Cu) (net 4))
 (segment (start 135.89 113.3475) (end 131.7625 117.475) (width 0.5) (layer F.Cu) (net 4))
 (segment (start 131.7625 117.475) (end 131.445 117.475) (width 0.5) (layer F.Cu) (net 4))
 (segment (start 154.94 139.7) (end 154.94 137.16) (width 0.5) (layer F.Cu) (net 5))
 (segment (start 154.94 137.16) (end 161.29 130.81) (width 0.5) (layer F.Cu) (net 5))
 (segment (start 149.82 134.62) (end 154.9 139.7) (width 0.5) (layer F.Cu) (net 5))
 (segment (start 154.9 139.7) (end 154.94 139.7) (width 0.5) (layer F.Cu) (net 5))
 (segment (start 154.94 142.24) (end 156.190001 140.989999) (width 0.5) (layer F.Cu) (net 6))
 (segment (start 156.190001 140.989999) (end 156.190001 138.449999) (width 0.5) (layer F.Cu) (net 6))
 (segment (start 156.190001 138.449999) (end 160.490001 134.149999) (width 0.5) (layer F.Cu) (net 6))
 (segment (start 160.490001 134.149999) (end 161.29 133.35) (width 0.5) (layer F.Cu) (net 6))
 (segment (start 138.47 134.62) (end 146.09 142.24) (width 0.5) (layer F.Cu) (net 6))
 (segment (start 146.09 142.24) (end 154.94 142.24) (width 0.5) (layer F.Cu) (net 6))
 (segment (start 156.21 115.57) (end 161.29 110.49) (width 0.5) (layer F.Cu) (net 7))
 (segment (start 156.21 120.65) (end 156.21 115.57) (width 0.5) (layer F.Cu) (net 7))
 (segment (start 152 120.65) (end 152 116.994002) (width 0.5) (layer F.Cu) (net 18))
 (segment (start 159.494001 109.500001) (end 159.739999 109.500001) (width 0.5) (layer F.Cu) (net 18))
 (segment (start 152 116.994002) (end 159.494001 109.500001) (width 0.5) (layer F.Cu) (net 18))
 (segment (start 168.110001 122.390001) (end 168.91 123.19) (width 0.5) (layer F.Cu) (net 18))
 (segment (start 164.359966 118.639966) (end 168.110001 122.390001) (width 0.5) (layer F.Cu) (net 18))
 (segment (start 164.359966 110.609964) (end 164.359966 118.639966) (width 0.5) (layer F.Cu) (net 18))
 (segment (start 162.690001 108.939999) (end 164.359966 110.609964) (width 0.5) (layer F.Cu) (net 18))
 (segment (start 159.889999 108.939999) (end 162.690001 108.939999) (width 0.5) (layer F.Cu) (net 18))
 (segment (start 159.739999 109.089999) (end 159.889999 108.939999) (width 0.5) (layer F.Cu) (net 18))
 (segment (start 159.739999 109.500001) (end 159.739999 109.089999) (width 0.5) (layer F.Cu) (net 18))
 (segment (start 180.34 133.35) (end 179.540001 132.550001) (width 0.5) (layer F.Cu) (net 18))
 (segment (start 179.540001 132.550001) (end 179.540001 131.525999) (width 0.5) (layer F.Cu) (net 18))
 (segment (start 179.540001 131.525999) (end 171.204002 123.19) (width 0.5) (layer F.Cu) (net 18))
 (segment (start 171.204002 123.19) (end 170.04137 123.19) (width 0.5) (layer F.Cu) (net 18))
 (segment (start 170.04137 123.19) (end 168.91 123.19) (width 0.5) (layer F.Cu) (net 18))
 (segment (start 148 120.38) (end 148 118.7) (width 0.5) (layer F.Cu) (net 19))
 (segment (start 148 118.7) (end 154.94 111.76) (width 0.5) (layer F.Cu) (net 19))
 (segment (start 168.110001 119.850001) (end 168.91 120.65) (width 0.5) (layer F.Cu) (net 19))
 (segment (start 163.104219 107.939988) (end 165.359977 110.195746) (width 0.5) (layer F.Cu) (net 19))
 (segment (start 158.760012 107.939988) (end 163.104219 107.939988) (width 0.5) (layer F.Cu) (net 19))
 (segment (start 154.94 111.76) (end 158.760012 107.939988) (width 0.5) (layer F.Cu) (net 19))
 (segment (start 165.359977 110.195746) (end 165.359977 117.099977) (width 0.5) (layer F.Cu) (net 19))
 (segment (start 165.359977 117.099977) (end 168.110001 119.850001) (width 0.5) (layer F.Cu) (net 19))
 (segment (start 170.04137 120.65) (end 168.91 120.65) (width 0.5) (layer F.Cu) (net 19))
 (segment (start 138.503998 107) (end 157.405998 107) (width 0.5) (layer F.Cu) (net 21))
 (segment (start 157.405998 107) (end 157.466021 106.939977) (width 0.5) (layer F.Cu) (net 21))
 (segment (start 131.445 118.745) (end 130.3735 118.745) (width 0.5) (layer F.Cu) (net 21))
 (segment (start 130.3735 118.745) (end 130.123499 118.494999) (width 0.5) (layer F.Cu) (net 21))
 (segment (start 130.123499 118.494999) (end 130.123499 115.380499) (width 0.5) (layer F.Cu) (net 21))
 (segment (start 130.123499 115.380499) (end 138.503998 107) (width 0.5) (layer F.Cu) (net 21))
 (segment (start 168.110001 117.310001) (end 168.91 118.11) (width 0.5) (layer F.Cu) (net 21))
 (segment (start 166.359988 115.559988) (end 168.110001 117.310001) (width 0.5) (layer F.Cu) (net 21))
 (segment (start 166.359988 109.781528) (end 166.359988 115.559988) (width 0.5) (layer F.Cu) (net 21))
 (segment (start 157.466021 106.939977) (end 163.518437 106.939977) (width 0.5) (layer F.Cu) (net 21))
 (segment (start 163.518437 106.939977) (end 166.359988 109.781528) (width 0.5) (layer F.Cu) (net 21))
 (segment (start 170.460001 113.430001) (end 170.460001 109.745999) (width 0.5) (layer F.Cu) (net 23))
 (segment (start 176.53 117.8) (end 174.83 117.8) (width 0.5) (layer F.Cu) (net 23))
 (segment (start 169.654001 108.939999) (end 168.165999 108.939999) (width 0.5) (layer F.Cu) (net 23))
 (segment (start 167.359999 109.745999) (end 167.359999 114.019999) (width 0.5) (layer F.Cu) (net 23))
 (segment (start 167.359999 114.019999) (end 168.110001 114.770001) (width 0.5) (layer F.Cu) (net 23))
 (segment (start 168.110001 114.770001) (end 168.91 115.57) (width 0.5) (layer F.Cu) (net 23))
 (segment (start 174.83 117.8) (end 170.460001 113.430001) (width 0.5) (layer F.Cu) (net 23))
 (segment (start 170.460001 109.745999) (end 169.654001 108.939999) (width 0.5) (layer F.Cu) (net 23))
 (segment (start 168.165999 108.939999) (end 167.359999 109.745999) (width 0.5) (layer F.Cu) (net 23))
 (segment (start 170.460001 115.480003) (end 170.460001 114.84423) (width 0.5) (layer F.Cu) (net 25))
 (segment (start 170.460001 114.84423) (end 168.91 113.294229) (width 0.5) (layer F.Cu) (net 25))
 (segment (start 168.91 113.294229) (end 168.91 113.03) (width 0.5) (layer F.Cu) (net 25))
 (segment (start 175.384003 119.750001) (end 174.729999 119.750001) (width 0.5) (layer F.Cu) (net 25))
 (segment (start 174.729999 119.750001) (end 170.460001 115.480003) (width 0.5) (layer F.Cu) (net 25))
 (segment (start 178.23 143.51) (end 180.999989 140.740011) (width 0.5) (layer F.Cu) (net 25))
 (segment (start 180.999989 140.740011) (end 180.999989 134.984013) (width 0.5) (layer F.Cu) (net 25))
 (segment (start 181.890001 127.744001) (end 181.890001 126.255999) (width 0.5) (layer F.Cu) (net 25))
 (segment (start 181.890001 126.255999) (end 175.384003 119.750001) (width 0.5) (layer F.Cu) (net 25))
 (segment (start 180.999989 128.634013) (end 181.890001 127.744001) (width 0.5) (layer F.Cu) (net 25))
 (segment (start 180.999989 131.799999) (end 180.999989 128.634013) (width 0.5) (layer F.Cu) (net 25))
 (segment (start 181.890001 132.690011) (end 180.999989 131.799999) (width 0.5) (layer F.Cu) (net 25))
 (segment (start 180.999989 134.984013) (end 181.890001 134.094001) (width 0.5) (layer F.Cu) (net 25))
 (segment (start 181.890001 134.094001) (end 181.890001 132.690011) (width 0.5) (layer F.Cu) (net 25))
 (segment (start 176.53 143.51) (end 178.23 143.51) (width 0.5) (layer F.Cu) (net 25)))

